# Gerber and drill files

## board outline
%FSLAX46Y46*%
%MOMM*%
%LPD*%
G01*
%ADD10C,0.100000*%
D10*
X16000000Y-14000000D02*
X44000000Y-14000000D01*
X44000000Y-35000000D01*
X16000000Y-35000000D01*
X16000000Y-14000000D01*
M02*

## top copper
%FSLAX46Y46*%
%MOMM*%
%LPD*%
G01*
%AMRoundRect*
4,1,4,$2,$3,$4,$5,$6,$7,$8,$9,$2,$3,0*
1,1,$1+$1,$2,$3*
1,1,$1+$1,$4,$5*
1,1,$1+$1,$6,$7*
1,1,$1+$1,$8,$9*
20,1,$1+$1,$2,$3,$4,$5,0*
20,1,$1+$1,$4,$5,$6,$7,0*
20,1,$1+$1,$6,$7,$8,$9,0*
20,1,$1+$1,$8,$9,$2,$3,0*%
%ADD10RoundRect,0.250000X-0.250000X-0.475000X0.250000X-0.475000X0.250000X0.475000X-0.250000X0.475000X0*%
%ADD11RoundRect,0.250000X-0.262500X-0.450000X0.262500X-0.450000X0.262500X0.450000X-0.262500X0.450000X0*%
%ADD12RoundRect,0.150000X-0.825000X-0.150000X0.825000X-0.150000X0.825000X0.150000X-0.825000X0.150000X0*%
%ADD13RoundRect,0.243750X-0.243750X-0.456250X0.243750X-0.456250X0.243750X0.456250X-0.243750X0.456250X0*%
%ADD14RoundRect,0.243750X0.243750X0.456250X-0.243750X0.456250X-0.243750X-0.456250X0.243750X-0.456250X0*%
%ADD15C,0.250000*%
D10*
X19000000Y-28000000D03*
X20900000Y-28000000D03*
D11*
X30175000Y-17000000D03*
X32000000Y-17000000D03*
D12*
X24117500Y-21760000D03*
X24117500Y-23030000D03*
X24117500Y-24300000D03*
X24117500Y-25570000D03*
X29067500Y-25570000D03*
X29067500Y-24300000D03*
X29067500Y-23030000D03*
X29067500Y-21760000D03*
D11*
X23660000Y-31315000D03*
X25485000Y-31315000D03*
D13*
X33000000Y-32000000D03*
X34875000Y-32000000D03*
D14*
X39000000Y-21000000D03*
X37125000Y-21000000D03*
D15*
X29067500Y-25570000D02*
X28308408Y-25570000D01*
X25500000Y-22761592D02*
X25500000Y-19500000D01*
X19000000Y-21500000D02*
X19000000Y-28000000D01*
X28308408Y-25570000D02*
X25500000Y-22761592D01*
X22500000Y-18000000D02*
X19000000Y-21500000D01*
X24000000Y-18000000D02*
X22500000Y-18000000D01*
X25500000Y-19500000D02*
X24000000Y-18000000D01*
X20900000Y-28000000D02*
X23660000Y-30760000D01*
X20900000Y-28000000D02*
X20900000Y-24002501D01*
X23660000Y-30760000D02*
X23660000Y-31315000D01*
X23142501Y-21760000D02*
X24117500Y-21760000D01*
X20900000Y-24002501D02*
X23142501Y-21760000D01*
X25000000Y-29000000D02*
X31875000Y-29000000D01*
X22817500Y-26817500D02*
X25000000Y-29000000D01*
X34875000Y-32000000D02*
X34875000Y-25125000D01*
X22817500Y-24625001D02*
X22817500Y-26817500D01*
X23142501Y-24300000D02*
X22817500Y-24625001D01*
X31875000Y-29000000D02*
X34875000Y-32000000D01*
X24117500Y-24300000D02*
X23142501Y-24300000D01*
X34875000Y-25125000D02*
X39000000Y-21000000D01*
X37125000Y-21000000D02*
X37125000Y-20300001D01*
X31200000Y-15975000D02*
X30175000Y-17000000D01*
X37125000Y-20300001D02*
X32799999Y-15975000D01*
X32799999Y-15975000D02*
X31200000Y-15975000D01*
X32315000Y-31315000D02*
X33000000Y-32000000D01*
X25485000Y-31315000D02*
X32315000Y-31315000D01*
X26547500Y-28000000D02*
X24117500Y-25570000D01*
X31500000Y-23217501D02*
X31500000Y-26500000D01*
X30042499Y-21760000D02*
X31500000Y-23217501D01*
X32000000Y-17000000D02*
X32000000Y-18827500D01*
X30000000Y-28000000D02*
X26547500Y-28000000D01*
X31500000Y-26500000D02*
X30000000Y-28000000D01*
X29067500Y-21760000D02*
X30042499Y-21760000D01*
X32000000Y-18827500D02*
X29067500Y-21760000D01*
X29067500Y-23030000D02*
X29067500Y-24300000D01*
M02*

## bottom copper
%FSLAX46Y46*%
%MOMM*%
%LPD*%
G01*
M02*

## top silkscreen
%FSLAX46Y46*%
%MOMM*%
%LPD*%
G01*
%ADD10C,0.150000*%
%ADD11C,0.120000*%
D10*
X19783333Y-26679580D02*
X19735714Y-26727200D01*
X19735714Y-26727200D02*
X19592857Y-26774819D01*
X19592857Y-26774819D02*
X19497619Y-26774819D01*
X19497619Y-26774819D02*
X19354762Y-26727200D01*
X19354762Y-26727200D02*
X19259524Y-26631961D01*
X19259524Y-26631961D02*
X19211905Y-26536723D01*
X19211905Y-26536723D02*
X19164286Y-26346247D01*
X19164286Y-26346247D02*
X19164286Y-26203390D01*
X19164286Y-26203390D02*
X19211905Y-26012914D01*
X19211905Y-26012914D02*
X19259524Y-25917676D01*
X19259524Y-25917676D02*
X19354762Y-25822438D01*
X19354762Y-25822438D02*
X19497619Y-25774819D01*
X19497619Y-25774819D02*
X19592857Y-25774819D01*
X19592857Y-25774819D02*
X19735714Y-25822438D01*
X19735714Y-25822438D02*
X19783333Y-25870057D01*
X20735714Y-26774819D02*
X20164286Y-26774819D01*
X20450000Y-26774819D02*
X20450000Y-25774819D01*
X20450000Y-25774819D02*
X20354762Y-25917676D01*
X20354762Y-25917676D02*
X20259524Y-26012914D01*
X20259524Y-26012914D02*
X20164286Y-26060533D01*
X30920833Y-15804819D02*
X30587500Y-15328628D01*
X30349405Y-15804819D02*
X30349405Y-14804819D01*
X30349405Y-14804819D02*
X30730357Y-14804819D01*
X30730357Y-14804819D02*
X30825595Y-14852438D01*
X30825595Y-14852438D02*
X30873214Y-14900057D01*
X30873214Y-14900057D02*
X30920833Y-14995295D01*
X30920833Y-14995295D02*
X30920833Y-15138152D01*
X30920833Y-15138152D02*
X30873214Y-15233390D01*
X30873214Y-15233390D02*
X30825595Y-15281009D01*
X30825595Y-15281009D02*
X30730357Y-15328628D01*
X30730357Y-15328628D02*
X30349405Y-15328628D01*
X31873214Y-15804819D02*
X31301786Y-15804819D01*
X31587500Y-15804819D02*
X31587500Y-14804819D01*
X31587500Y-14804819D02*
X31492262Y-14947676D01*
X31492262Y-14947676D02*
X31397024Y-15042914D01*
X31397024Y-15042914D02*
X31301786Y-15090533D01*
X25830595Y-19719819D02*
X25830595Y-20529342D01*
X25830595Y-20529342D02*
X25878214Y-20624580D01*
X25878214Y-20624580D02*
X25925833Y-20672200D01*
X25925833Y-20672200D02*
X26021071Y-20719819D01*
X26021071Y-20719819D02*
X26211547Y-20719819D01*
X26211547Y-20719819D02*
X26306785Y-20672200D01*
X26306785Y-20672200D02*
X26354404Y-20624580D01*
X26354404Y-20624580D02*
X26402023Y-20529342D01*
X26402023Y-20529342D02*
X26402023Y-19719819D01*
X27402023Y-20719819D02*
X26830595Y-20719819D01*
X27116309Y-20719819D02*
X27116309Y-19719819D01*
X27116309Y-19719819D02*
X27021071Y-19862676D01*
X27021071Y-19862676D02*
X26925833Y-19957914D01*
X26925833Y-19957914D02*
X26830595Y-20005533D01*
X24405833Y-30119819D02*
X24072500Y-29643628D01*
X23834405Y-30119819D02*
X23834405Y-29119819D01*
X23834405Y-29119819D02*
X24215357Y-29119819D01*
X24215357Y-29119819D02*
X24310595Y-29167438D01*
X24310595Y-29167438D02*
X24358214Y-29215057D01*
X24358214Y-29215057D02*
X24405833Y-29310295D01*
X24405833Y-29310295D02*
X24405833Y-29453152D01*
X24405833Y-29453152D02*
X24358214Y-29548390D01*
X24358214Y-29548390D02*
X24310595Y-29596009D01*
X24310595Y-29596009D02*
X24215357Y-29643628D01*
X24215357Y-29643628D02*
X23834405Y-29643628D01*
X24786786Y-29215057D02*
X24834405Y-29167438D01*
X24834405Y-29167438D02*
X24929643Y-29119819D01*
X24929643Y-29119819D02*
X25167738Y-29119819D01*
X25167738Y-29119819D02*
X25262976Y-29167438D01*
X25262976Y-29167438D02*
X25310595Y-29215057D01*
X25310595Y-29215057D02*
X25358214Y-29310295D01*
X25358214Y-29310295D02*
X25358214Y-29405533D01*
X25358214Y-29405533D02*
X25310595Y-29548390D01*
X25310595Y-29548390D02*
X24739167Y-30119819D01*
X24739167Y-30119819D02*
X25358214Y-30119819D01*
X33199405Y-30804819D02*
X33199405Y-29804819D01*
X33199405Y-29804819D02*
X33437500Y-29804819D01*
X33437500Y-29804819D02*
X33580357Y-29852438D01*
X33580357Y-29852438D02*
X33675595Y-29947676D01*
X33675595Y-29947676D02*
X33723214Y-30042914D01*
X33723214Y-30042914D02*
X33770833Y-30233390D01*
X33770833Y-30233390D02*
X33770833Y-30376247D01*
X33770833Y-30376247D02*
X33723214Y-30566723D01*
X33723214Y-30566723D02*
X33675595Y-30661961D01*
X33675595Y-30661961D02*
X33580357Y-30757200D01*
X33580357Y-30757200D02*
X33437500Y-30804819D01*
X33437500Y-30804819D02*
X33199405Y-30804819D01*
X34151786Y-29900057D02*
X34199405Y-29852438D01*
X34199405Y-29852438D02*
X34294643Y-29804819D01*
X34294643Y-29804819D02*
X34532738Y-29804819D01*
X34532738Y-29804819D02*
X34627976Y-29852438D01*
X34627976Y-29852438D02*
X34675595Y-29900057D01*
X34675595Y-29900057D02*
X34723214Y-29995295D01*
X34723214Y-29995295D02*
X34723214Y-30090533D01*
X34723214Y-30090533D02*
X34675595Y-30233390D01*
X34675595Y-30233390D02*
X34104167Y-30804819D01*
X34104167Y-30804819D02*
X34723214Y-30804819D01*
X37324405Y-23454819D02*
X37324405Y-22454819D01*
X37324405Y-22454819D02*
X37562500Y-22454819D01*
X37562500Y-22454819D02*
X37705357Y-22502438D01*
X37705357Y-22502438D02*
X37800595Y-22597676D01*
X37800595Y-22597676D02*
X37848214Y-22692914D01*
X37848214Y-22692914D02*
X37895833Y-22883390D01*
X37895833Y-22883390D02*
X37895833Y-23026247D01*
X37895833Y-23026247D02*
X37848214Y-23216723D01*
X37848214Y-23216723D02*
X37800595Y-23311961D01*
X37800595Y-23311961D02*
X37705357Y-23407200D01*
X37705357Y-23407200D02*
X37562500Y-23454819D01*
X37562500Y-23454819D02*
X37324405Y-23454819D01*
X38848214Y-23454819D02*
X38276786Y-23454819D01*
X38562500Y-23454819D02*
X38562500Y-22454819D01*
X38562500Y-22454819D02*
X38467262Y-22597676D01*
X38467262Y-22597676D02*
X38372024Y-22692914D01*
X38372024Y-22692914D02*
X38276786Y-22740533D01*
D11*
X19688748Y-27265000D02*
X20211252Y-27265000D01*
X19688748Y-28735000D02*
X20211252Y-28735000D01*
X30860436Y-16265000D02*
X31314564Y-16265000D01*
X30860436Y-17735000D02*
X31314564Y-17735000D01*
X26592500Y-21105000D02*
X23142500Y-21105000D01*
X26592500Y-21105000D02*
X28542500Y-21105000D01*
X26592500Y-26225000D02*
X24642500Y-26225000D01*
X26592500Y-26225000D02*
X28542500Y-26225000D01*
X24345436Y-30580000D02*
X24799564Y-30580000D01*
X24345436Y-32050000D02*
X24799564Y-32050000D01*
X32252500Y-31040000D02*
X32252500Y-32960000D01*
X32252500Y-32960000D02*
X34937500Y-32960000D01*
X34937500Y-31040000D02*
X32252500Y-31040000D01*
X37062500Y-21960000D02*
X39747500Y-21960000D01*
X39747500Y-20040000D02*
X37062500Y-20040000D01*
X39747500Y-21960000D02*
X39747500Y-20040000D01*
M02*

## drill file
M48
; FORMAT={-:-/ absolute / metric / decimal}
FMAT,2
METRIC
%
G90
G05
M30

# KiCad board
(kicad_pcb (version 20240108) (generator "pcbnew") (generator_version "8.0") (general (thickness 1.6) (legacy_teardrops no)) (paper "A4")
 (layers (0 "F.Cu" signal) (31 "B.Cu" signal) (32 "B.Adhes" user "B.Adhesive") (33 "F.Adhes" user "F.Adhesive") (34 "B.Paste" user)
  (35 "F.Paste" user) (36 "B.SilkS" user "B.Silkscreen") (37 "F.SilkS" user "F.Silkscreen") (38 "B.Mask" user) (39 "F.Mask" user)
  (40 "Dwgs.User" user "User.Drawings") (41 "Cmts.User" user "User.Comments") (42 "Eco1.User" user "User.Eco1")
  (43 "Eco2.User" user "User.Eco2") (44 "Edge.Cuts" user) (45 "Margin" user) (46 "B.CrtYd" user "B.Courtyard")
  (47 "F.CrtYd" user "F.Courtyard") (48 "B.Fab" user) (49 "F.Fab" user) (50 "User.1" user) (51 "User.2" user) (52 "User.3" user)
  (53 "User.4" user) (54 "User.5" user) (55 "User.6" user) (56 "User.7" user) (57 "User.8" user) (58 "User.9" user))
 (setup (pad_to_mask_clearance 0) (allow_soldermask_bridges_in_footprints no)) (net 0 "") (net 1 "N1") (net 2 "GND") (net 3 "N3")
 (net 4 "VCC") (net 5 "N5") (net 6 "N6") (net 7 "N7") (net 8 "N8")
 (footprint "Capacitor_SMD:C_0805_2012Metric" (layer "F.Cu") (at 19.95 28)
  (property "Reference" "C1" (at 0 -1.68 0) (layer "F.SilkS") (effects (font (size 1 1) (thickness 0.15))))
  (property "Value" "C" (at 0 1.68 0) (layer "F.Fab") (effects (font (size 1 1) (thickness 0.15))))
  (fp_line (start -0.261252 -0.735) (end 0.261252 -0.735) (stroke (width 0.12) (type solid)) (layer "F.SilkS"))
  (fp_line (start -0.261252 0.735) (end 0.261252 0.735) (stroke (width 0.12) (type solid)) (layer "F.SilkS"))
  (pad "1" smd roundrect (at -0.95 0) (size 1 1.45) (layers "F.Cu" "F.Paste" "F.Mask") (roundrect_rratio 0.25) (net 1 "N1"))
  (pad "2" smd roundrect (at 0.95 0) (size 1 1.45) (layers "F.Cu" "F.Paste" "F.Mask") (roundrect_rratio 0.25) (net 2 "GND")))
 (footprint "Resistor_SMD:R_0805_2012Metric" (layer "F.Cu") (at 31.0875 17)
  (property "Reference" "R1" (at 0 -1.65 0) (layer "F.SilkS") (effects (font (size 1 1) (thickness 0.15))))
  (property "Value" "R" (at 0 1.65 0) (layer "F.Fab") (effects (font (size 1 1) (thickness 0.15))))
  (fp_line (start -0.227064 -0.735) (end 0.227064 -0.735) (stroke (width 0.12) (type solid)) (layer "F.SilkS"))
  (fp_line (start -0.227064 0.735) (end 0.227064 0.735) (stroke (width 0.12) (type solid)) (layer "F.SilkS"))
  (pad "1" smd roundrect (at -0.9125 0) (size 1.025 1.4) (layers "F.Cu" "F.Paste" "F.Mask") (roundrect_rratio 0.243902) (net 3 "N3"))
  (pad "2" smd roundrect (at 0.9125 0) (size 1.025 1.4) (layers "F.Cu" "F.Paste" "F.Mask") (roundrect_rratio 0.243902) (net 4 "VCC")))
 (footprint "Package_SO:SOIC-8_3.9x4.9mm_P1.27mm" (layer "F.Cu") (at 26.5925 23.665)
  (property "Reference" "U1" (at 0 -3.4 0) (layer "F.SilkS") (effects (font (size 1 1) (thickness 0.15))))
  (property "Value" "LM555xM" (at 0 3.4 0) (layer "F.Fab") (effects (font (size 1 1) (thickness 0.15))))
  (fp_line (start 0 -2.56) (end -3.45 -2.56) (stroke (width 0.12) (type solid)) (layer "F.SilkS"))
  (fp_line (start 0 -2.56) (end 1.95 -2.56) (stroke (width 0.12) (type solid)) (layer "F.SilkS"))
  (fp_line (start 0 2.56) (end -1.95 2.56) (stroke (width 0.12) (type solid)) (layer "F.SilkS"))
  (fp_line (start 0 2.56) (end 1.95 2.56) (stroke (width 0.12) (type solid)) (layer "F.SilkS"))
  (pad "1" smd roundrect (at -2.475 -1.905) (size 1.95 0.6) (layers "F.Cu" "F.Paste" "F.Mask") (roundrect_rratio 0.25) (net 2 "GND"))
  (pad "2" smd roundrect (at -2.475 -0.635) (size 1.95 0.6) (layers "F.Cu" "F.Paste" "F.Mask") (roundrect_rratio 0.25) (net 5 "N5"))
  (pad "3" smd roundrect (at -2.475 0.635) (size 1.95 0.6) (layers "F.Cu" "F.Paste" "F.Mask") (roundrect_rratio 0.25) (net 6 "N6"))
  (pad "4" smd roundrect (at -2.475 1.905) (size 1.95 0.6) (layers "F.Cu" "F.Paste" "F.Mask") (roundrect_rratio 0.25) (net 4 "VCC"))
  (pad "5" smd roundrect (at 2.475 1.905) (size 1.95 0.6) (layers "F.Cu" "F.Paste" "F.Mask") (roundrect_rratio 0.25) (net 1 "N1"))
  (pad "6" smd roundrect (at 2.475 0.635) (size 1.95 0.6) (layers "F.Cu" "F.Paste" "F.Mask") (roundrect_rratio 0.25) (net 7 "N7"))
  (pad "7" smd roundrect (at 2.475 -0.635) (size 1.95 0.6) (layers "F.Cu" "F.Paste" "F.Mask") (roundrect_rratio 0.25) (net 7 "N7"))
  (pad "8" smd roundrect (at 2.475 -1.905) (size 1.95 0.6) (layers "F.Cu" "F.Paste" "F.Mask") (roundrect_rratio 0.25) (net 4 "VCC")))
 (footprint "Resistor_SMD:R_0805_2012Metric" (layer "F.Cu") (at 24.5725 31.315)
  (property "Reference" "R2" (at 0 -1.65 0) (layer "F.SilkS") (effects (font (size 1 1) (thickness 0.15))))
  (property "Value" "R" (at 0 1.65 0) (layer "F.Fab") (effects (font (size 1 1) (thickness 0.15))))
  (fp_line (start -0.227064 -0.735) (end 0.227064 -0.735) (stroke (width 0.12) (type solid)) (layer "F.SilkS"))
  (fp_line (start -0.227064 0.735) (end 0.227064 0.735) (stroke (width 0.12) (type solid)) (layer "F.SilkS"))
  (pad "1" smd roundrect (at -0.9125 0) (size 1.025 1.4) (layers "F.Cu" "F.Paste" "F.Mask") (roundrect_rratio 0.243902) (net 2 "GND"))
  (pad "2" smd roundrect (at 0.9125 0) (size 1.025 1.4) (layers "F.Cu" "F.Paste" "F.Mask") (roundrect_rratio 0.243902) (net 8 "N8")))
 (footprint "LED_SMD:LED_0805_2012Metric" (layer "F.Cu") (at 33.9375 32)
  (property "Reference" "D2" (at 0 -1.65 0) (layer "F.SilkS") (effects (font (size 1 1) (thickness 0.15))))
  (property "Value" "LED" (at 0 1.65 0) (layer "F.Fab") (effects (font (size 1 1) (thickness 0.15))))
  (fp_line (start -1.685 -0.96) (end -1.685 0.96) (stroke (width 0.12) (type solid)) (layer "F.SilkS"))
  (fp_line (start -1.685 0.96) (end 1 0.96) (stroke (width 0.12) (type solid)) (layer "F.SilkS"))
  (fp_line (start 1 -0.96) (end -1.685 -0.96) (stroke (width 0.12) (type solid)) (layer "F.SilkS"))
  (pad "1" smd roundrect (at -0.9375 0) (size 0.975 1.4) (layers "F.Cu" "F.Paste" "F.Mask") (roundrect_rratio 0.25) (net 8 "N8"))
  (pad "2" smd roundrect (at 0.9375 0) (size 0.975 1.4) (layers "F.Cu" "F.Paste" "F.Mask") (roundrect_rratio 0.25) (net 6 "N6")))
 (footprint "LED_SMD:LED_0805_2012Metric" (layer "F.Cu") (at 38.0625 21 180)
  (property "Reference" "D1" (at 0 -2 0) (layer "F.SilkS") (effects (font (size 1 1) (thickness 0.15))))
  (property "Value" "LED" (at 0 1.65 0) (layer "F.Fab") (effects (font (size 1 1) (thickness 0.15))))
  (fp_line (start 1 -0.96) (end -1.685 -0.96) (stroke (width 0.12) (type solid)) (layer "F.SilkS"))
  (fp_line (start -1.685 0.96) (end 1 0.96) (stroke (width 0.12) (type solid)) (layer "F.SilkS"))
  (fp_line (start -1.685 -0.96) (end -1.685 0.96) (stroke (width 0.12) (type solid)) (layer "F.SilkS"))
  (pad "1" smd roundrect (at -0.9375 0 180) (size 0.975 1.4) (layers "F.Cu" "F.Paste" "F.Mask") (roundrect_rratio 0.25) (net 6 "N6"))
  (pad "2" smd roundrect (at 0.9375 0 180) (size 0.975 1.4) (layers "F.Cu" "F.Paste" "F.Mask") (roundrect_rratio 0.25) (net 3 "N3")))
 (gr_rect (start 16 14) (end 44 35) (stroke (width 0.1) (type default)) (fill none) (layer "Edge.Cuts"))
 (segment (start 29.0675 25.57) (end 28.308408 25.57) (width 0.25) (layer "F.Cu") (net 1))
 (segment (start 25.5 22.761592) (end 25.5 19.5) (width 0.25) (layer "F.Cu") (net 1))
 (segment (start 19 21.5) (end 19 28) (width 0.25) (layer "F.Cu") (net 1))
 (segment (start 28.308408 25.57) (end 25.5 22.761592) (width 0.25) (layer "F.Cu") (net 1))
 (segment (start 22.5 18) (end 19 21.5) (width 0.25) (layer "F.Cu") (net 1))
 (segment (start 24 18) (end 22.5 18) (width 0.25) (layer "F.Cu") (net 1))
 (segment (start 25.5 19.5) (end 24 18) (width 0.25) (layer "F.Cu") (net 1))
 (segment (start 20.9 28) (end 23.66 30.76) (width 0.25) (layer "F.Cu") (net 2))
 (segment (start 20.9 28) (end 20.9 24.002501) (width 0.25) (layer "F.Cu") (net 2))
 (segment (start 23.66 30.76) (end 23.66 31.315) (width 0.25) (layer "F.Cu") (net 2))
 (segment (start 23.142501 21.76) (end 24.1175 21.76) (width 0.25) (layer "F.Cu") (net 2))
 (segment (start 20.9 24.002501) (end 23.142501 21.76) (width 0.25) (layer "F.Cu") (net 2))
 (segment (start 25 29) (end 31.875 29) (width 0.25) (layer "F.Cu") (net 6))
 (segment (start 22.8175 26.8175) (end 25 29) (width 0.25) (layer "F.Cu") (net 6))
 (segment (start 34.875 32) (end 34.875 25.125) (width 0.25) (layer "F.Cu") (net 6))
 (segment (start 22.8175 24.625001) (end 22.8175 26.8175) (width 0.25) (layer "F.Cu") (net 6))
 (segment (start 23.142501 24.3) (end 22.8175 24.625001) (width 0.25) (layer "F.Cu") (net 6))
 (segment (start 31.875 29) (end 34.875 32) (width 0.25) (layer "F.Cu") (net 6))
 (segment (start 24.1175 24.3) (end 23.142501 24.3) (width 0.25) (layer "F.Cu") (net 6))
 (segment (start 34.875 25.125) (end 39 21) (width 0.25) (layer "F.Cu") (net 6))
 (segment (start 37.125 21) (end 37.125 20.300001) (width 0.25) (layer "F.Cu") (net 3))
 (segment (start 31.2 15.975) (end 30.175 17) (width 0.25) (layer "F.Cu") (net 3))
 (segment (start 37.125 20.300001) (end 32.799999 15.975) (width 0.25) (layer "F.Cu") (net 3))
 (segment (start 32.799999 15.975) (end 31.2 15.975) (width 0.25) (layer "F.Cu") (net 3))
 (segment (start 32.315 31.315) (end 33 32) (width 0.25) (layer "F.Cu") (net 8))
 (segment (start 25.485 31.315) (end 32.315 31.315) (width 0.25) (layer "F.Cu") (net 8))
 (segment (start 26.5475 28) (end 24.1175 25.57) (width 0.25) (layer "F.Cu") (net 4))
 (segment (start 31.5 23.217501) (end 31.5 26.5) (width 0.25) (layer "F.Cu") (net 4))
 (segment (start 30.042499 21.76) (end 31.5 23.217501) (width 0.25) (layer "F.Cu") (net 4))
 (segment (start 32 17) (end 32 18.8275) (width 0.25) (layer "F.Cu") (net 4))
 (segment (start 30 28) (end 26.5475 28) (width 0.25) (layer "F.Cu") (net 4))
 (segment (start 31.5 26.5) (end 30 28) (width 0.25) (layer "F.Cu") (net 4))
 (segment (start 29.0675 21.76) (end 30.042499 21.76) (width 0.25) (layer "F.Cu") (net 4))
 (segment (start 32 18.8275) (end 29.0675 21.76) (width 0.25) (layer "F.Cu") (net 4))
 (segment (start 29.0675 23.03) (end 29.0675 24.3) (width 0.25) (layer "F.Cu") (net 7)))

